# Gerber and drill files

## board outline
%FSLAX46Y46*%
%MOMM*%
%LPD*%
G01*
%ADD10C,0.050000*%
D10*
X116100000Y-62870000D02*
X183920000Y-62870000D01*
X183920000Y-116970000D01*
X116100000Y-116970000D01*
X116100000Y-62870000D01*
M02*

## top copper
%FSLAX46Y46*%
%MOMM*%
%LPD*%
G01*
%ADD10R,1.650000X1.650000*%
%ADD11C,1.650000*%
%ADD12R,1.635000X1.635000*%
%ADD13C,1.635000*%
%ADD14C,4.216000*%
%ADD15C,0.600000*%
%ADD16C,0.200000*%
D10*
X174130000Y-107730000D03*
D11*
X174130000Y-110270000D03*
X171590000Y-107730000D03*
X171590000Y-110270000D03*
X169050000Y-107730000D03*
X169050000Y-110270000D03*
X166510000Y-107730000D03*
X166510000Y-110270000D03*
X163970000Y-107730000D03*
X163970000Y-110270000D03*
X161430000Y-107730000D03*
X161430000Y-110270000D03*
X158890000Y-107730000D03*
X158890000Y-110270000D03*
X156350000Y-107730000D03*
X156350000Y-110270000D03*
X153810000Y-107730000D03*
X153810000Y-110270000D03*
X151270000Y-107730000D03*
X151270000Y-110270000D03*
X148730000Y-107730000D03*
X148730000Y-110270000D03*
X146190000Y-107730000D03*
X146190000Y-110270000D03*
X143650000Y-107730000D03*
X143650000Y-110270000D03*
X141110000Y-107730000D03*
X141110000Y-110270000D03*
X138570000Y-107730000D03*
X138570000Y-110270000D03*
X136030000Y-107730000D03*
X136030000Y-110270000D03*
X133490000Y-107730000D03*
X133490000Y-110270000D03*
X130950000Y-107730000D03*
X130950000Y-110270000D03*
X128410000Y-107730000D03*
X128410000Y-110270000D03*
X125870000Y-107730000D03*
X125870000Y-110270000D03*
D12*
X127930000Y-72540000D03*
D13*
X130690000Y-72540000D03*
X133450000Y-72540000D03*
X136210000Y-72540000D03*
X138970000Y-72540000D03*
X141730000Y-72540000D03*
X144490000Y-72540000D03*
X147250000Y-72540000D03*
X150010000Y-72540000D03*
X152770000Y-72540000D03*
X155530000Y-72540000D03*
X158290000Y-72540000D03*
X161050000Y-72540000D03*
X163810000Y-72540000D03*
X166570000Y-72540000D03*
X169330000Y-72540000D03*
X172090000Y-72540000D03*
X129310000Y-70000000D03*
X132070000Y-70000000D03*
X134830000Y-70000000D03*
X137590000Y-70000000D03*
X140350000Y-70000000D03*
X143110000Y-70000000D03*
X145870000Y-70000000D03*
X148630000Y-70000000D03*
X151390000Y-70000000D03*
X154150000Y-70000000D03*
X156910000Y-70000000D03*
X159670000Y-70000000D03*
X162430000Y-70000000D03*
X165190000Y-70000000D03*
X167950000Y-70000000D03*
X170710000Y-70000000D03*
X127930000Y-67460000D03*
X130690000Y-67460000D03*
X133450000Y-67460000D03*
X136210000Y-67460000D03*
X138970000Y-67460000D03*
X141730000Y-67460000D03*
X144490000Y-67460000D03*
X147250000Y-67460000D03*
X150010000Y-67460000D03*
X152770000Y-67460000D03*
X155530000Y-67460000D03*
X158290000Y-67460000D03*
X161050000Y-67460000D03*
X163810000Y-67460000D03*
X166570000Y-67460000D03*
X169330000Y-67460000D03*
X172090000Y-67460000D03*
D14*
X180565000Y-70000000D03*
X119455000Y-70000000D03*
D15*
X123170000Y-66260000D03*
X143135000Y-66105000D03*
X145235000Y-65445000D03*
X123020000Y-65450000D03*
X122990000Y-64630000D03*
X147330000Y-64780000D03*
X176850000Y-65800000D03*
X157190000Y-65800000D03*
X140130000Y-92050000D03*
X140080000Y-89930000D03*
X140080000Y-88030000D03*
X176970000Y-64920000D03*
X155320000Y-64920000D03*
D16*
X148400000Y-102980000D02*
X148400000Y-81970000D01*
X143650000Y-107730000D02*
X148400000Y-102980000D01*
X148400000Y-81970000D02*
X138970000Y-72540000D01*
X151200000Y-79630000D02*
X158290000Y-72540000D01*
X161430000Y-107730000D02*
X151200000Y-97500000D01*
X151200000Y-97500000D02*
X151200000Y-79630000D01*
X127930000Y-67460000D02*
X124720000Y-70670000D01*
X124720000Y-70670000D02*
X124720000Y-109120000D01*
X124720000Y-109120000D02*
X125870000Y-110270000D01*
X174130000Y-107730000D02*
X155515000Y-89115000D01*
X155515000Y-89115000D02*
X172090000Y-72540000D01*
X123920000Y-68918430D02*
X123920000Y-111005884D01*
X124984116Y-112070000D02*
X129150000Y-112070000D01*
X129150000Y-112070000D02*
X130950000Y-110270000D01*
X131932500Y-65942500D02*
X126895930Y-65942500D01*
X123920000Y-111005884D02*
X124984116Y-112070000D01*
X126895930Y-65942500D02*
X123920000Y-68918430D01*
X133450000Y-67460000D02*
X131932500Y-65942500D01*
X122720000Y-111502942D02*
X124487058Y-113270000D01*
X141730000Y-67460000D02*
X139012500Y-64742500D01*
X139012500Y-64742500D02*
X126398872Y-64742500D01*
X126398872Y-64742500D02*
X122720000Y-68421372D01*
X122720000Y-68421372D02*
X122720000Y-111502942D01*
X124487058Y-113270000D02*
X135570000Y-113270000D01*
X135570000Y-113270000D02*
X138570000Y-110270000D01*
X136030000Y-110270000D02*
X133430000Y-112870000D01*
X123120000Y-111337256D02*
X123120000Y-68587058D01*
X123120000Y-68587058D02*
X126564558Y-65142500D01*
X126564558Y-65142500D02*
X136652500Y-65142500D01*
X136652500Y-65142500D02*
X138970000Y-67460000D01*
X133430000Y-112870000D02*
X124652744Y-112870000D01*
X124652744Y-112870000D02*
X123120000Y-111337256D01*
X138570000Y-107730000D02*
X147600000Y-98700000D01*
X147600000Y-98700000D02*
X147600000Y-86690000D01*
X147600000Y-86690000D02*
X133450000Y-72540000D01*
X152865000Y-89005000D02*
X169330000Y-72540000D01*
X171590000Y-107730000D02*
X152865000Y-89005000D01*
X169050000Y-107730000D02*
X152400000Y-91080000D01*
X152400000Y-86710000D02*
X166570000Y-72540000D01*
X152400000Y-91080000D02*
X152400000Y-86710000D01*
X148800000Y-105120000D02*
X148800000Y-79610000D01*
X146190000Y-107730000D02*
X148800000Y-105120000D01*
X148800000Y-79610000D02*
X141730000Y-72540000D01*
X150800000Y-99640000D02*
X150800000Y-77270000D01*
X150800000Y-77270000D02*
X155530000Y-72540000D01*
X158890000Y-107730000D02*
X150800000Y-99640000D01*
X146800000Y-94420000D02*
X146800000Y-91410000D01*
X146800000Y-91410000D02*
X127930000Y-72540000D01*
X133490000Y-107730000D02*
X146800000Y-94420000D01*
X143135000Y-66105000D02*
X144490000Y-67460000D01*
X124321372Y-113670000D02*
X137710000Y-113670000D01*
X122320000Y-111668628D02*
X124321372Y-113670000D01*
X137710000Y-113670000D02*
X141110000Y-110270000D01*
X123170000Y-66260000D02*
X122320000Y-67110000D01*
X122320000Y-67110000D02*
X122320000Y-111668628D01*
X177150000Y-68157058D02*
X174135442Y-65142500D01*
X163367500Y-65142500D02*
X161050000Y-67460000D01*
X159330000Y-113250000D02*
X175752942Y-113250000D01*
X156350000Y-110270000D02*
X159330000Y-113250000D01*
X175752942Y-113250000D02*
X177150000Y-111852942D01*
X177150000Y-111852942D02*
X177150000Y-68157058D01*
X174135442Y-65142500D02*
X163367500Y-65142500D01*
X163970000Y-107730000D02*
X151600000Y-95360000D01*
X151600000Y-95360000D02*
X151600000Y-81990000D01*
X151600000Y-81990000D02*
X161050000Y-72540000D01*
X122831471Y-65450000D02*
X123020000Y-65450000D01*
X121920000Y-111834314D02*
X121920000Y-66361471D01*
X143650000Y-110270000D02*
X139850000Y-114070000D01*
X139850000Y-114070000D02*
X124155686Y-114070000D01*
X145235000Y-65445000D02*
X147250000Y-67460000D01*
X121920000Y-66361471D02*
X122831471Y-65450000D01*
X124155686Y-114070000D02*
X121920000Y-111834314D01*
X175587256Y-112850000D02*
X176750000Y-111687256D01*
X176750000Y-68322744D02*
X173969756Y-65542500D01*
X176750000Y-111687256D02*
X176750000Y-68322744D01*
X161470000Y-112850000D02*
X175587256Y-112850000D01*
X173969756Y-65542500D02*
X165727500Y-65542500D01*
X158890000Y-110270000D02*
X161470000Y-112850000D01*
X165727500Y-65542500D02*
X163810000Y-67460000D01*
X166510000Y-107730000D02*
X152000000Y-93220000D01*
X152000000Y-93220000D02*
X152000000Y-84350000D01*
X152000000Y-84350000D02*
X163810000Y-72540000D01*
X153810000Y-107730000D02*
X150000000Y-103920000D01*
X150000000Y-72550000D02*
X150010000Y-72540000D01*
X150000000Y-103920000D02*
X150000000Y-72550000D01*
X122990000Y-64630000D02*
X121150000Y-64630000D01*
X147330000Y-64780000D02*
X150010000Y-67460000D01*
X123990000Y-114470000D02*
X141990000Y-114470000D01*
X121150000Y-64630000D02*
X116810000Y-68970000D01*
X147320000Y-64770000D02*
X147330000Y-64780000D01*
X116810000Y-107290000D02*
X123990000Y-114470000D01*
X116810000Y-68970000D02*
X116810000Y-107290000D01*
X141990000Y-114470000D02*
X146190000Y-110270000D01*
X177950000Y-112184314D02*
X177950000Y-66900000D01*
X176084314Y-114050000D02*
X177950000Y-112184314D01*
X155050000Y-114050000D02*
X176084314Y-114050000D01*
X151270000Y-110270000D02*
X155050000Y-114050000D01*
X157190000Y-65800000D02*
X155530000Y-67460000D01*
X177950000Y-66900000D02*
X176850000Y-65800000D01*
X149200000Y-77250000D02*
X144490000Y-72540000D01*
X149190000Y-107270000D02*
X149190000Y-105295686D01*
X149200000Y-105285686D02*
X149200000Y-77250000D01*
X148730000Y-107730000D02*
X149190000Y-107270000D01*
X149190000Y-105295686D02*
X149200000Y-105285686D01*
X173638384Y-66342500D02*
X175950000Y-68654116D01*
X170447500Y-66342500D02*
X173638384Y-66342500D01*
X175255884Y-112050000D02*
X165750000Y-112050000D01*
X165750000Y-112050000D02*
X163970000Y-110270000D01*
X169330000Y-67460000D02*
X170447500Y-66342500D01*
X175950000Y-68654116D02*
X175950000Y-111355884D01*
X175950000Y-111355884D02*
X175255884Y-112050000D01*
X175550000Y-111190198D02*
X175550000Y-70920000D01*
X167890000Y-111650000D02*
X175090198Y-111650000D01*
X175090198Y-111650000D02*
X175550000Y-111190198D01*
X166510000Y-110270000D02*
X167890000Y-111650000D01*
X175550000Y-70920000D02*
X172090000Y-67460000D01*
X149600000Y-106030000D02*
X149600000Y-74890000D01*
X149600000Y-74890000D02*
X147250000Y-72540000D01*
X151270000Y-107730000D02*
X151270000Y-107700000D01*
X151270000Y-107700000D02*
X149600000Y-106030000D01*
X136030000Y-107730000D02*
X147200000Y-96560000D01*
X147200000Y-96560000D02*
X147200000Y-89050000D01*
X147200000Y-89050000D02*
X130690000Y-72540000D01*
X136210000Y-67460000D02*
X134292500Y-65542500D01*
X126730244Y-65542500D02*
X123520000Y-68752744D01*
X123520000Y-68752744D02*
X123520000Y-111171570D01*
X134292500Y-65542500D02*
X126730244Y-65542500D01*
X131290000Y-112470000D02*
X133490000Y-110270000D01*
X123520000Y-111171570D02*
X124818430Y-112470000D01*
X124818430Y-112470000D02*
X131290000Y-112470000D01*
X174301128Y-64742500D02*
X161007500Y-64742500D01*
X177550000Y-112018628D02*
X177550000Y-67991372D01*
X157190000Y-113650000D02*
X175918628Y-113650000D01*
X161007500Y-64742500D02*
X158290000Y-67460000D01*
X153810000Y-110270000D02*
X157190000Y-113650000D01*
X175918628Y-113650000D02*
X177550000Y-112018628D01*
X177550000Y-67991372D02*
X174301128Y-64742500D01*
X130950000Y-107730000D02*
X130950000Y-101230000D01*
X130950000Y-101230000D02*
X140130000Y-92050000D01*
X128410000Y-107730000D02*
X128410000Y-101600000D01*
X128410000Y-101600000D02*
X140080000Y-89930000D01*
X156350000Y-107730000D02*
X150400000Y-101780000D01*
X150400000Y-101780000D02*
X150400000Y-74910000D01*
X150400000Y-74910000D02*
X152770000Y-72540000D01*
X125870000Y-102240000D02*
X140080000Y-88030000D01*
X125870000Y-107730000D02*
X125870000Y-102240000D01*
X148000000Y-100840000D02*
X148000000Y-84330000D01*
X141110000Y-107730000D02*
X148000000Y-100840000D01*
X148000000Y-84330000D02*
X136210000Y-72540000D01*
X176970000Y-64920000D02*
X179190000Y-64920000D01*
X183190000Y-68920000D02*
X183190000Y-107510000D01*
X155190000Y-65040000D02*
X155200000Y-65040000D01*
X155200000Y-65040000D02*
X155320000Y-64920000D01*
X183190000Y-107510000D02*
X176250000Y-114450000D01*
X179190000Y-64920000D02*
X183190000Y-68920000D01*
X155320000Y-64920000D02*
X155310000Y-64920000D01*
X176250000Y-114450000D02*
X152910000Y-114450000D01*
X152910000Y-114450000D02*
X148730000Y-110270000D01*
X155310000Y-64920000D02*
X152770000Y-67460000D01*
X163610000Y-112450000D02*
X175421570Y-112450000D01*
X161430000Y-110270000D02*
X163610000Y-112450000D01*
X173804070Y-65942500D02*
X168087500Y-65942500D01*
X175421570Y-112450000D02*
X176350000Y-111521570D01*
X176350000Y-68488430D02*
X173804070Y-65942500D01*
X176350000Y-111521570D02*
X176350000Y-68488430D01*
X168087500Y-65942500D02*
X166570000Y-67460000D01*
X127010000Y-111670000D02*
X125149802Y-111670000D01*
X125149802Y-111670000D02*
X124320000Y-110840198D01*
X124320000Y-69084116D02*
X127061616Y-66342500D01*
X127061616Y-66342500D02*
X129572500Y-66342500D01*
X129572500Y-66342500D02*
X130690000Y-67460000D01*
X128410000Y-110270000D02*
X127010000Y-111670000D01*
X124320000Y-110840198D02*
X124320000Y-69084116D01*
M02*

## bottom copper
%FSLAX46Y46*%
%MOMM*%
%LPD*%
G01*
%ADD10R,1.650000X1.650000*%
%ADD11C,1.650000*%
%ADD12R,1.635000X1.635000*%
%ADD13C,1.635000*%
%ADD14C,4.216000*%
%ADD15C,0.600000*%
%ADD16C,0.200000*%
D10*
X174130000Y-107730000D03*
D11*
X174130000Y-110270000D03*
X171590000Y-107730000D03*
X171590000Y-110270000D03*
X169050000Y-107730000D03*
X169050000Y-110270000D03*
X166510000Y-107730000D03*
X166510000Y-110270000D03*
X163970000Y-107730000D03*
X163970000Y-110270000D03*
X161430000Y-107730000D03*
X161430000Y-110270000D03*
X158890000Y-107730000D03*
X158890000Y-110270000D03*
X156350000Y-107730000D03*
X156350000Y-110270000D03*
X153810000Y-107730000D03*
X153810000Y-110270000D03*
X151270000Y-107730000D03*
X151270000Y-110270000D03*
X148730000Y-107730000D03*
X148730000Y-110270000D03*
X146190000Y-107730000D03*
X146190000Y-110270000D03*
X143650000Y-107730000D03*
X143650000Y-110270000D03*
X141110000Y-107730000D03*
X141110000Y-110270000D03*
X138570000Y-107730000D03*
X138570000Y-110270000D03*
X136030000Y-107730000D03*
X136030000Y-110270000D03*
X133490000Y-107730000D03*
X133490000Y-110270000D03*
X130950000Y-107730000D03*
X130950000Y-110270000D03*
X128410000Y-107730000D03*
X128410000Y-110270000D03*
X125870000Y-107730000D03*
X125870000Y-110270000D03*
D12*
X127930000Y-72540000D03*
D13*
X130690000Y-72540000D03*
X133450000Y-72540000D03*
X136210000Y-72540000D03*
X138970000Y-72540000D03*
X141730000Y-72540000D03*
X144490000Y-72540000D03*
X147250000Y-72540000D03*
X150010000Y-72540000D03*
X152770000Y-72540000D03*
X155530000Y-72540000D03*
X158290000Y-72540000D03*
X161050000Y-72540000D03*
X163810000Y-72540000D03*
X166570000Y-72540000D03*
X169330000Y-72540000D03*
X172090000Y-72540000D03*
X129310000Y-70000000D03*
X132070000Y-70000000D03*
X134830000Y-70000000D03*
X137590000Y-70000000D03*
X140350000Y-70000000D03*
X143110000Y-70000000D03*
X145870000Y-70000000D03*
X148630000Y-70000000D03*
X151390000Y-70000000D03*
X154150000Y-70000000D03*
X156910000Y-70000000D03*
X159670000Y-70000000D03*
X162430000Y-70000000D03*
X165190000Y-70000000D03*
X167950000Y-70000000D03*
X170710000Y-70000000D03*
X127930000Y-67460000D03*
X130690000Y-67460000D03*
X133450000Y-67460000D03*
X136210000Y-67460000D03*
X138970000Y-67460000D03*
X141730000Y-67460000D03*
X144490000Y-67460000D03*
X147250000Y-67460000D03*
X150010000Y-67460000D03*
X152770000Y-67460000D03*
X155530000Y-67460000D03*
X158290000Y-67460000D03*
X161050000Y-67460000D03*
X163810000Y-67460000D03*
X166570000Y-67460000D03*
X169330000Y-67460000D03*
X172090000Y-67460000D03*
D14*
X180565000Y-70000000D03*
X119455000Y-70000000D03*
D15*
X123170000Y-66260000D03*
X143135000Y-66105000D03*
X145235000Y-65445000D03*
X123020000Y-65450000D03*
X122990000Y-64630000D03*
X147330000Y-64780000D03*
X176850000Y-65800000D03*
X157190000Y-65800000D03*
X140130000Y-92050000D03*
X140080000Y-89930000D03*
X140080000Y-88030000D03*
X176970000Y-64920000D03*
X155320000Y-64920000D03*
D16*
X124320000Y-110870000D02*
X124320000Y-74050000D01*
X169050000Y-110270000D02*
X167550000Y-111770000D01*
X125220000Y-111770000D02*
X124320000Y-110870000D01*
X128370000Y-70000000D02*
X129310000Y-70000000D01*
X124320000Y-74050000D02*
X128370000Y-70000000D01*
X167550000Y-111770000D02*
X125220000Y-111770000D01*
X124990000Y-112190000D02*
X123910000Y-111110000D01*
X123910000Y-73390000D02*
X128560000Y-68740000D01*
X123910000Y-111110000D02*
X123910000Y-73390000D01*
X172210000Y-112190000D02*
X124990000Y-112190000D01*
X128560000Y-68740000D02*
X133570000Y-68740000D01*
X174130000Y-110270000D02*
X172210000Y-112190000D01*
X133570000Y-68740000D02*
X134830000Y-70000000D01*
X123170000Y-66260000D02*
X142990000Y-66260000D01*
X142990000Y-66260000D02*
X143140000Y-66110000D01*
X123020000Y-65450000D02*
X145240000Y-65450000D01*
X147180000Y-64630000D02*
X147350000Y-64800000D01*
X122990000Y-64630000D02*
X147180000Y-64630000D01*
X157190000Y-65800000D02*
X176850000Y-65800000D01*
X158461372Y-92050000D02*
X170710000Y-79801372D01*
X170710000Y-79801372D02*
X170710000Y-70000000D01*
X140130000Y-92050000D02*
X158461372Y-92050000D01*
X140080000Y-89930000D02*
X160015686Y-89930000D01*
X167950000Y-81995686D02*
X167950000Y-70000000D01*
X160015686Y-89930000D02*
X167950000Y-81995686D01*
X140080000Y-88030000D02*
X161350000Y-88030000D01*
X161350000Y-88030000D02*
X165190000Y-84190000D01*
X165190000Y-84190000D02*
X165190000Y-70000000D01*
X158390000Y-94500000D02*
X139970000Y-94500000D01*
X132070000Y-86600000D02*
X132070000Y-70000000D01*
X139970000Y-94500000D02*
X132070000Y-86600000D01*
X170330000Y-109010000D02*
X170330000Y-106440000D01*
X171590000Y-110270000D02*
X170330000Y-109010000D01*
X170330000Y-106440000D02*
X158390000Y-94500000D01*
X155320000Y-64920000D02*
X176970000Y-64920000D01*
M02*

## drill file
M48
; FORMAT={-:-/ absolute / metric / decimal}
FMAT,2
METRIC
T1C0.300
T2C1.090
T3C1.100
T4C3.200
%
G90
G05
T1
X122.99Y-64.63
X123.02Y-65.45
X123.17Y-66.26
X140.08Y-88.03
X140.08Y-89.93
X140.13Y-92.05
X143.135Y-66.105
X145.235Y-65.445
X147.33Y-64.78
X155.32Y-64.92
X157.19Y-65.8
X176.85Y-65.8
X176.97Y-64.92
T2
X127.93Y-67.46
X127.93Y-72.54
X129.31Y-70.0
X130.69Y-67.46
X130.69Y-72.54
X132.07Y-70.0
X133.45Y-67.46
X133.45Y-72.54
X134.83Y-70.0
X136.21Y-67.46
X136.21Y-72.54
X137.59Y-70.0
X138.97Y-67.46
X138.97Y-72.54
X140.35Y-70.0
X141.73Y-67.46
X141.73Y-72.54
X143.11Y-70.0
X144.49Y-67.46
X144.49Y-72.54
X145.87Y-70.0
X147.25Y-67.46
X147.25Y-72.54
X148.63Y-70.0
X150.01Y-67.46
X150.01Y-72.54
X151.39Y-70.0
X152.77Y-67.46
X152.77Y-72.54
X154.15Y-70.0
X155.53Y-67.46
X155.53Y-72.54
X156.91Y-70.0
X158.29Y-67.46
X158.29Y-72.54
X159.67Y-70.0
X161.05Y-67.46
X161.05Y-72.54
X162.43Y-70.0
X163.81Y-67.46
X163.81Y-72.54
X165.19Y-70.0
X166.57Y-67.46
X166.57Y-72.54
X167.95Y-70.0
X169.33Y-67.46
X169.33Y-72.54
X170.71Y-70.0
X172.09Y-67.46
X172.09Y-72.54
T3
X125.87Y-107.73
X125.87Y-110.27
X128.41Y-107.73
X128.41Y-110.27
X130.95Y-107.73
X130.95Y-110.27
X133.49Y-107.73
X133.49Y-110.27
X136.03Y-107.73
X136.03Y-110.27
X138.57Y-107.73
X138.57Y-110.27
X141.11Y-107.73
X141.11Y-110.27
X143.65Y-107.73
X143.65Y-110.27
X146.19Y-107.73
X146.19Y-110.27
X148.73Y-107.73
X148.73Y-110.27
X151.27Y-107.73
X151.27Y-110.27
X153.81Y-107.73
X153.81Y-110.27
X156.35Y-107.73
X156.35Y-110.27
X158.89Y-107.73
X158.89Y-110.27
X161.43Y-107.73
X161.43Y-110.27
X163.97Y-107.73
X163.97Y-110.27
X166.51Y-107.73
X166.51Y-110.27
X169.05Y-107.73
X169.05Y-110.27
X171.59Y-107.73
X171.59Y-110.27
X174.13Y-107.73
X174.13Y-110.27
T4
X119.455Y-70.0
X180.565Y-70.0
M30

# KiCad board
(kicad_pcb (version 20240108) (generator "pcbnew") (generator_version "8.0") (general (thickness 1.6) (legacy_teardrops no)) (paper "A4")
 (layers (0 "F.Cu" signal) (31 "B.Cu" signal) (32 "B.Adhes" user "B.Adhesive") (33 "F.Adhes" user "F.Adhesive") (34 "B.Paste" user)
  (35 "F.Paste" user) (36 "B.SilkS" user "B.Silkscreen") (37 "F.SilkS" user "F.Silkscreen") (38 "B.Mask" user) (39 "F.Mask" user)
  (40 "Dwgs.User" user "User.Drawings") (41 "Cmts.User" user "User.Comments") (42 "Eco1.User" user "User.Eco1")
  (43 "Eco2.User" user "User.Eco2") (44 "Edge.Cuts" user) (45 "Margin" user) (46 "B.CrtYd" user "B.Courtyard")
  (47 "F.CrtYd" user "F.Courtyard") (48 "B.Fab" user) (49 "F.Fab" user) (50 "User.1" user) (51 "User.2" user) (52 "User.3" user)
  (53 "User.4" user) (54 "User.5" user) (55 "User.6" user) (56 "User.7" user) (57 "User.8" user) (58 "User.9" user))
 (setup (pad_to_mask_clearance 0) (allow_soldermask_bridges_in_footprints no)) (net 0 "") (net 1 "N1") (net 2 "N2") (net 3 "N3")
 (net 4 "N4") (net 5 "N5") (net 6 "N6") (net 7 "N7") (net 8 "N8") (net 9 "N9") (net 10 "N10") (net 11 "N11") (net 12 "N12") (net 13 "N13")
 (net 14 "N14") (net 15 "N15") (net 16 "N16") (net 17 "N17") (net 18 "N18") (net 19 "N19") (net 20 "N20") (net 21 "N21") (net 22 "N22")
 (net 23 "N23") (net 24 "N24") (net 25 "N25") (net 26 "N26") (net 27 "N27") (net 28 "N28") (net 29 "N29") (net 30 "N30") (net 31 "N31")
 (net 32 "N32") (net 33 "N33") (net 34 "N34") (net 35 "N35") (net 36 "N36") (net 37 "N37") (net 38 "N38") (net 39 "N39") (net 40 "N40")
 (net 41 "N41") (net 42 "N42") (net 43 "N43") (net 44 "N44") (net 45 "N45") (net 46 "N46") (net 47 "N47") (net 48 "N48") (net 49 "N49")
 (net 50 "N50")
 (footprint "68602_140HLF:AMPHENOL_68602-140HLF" (layer "F.Cu") (at 150 109 180)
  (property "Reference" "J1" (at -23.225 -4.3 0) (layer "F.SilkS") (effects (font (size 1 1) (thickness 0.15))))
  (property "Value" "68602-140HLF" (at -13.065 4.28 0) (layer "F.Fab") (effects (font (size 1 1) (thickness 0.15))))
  (pad "01" thru_hole rect (at -24.13 1.27 180) (size 1.65 1.65) (drill 1.1) (layers "*.Cu" "*.Mask") (remove_unused_layers no) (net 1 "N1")
   (solder_mask_margin 0.102))
  (pad "02" thru_hole circle (at -24.13 -1.27 180) (size 1.65 1.65) (drill 1.1) (layers "*.Cu" "*.Mask") (remove_unused_layers no)
   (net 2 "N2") (solder_mask_margin 0.102))
  (pad "03" thru_hole circle (at -21.59 1.27 180) (size 1.65 1.65) (drill 1.1) (layers "*.Cu" "*.Mask") (remove_unused_layers no)
   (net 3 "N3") (solder_mask_margin 0.102))
  (pad "04" thru_hole circle (at -21.59 -1.27 180) (size 1.65 1.65) (drill 1.1) (layers "*.Cu" "*.Mask") (remove_unused_layers no)
   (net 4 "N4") (solder_mask_margin 0.102))
  (pad "05" thru_hole circle (at -19.05 1.27 180) (size 1.65 1.65) (drill 1.1) (layers "*.Cu" "*.Mask") (remove_unused_layers no)
   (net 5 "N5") (solder_mask_margin 0.102))
  (pad "06" thru_hole circle (at -19.05 -1.27 180) (size 1.65 1.65) (drill 1.1) (layers "*.Cu" "*.Mask") (remove_unused_layers no)
   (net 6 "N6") (solder_mask_margin 0.102))
  (pad "07" thru_hole circle (at -16.51 1.27 180) (size 1.65 1.65) (drill 1.1) (layers "*.Cu" "*.Mask") (remove_unused_layers no)
   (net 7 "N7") (solder_mask_margin 0.102))
  (pad "08" thru_hole circle (at -16.51 -1.27 180) (size 1.65 1.65) (drill 1.1) (layers "*.Cu" "*.Mask") (remove_unused_layers no)
   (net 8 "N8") (solder_mask_margin 0.102))
  (pad "09" thru_hole circle (at -13.97 1.27 180) (size 1.65 1.65) (drill 1.1) (layers "*.Cu" "*.Mask") (remove_unused_layers no)
   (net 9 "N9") (solder_mask_margin 0.102))
  (pad "10" thru_hole circle (at -13.97 -1.27 180) (size 1.65 1.65) (drill 1.1) (layers "*.Cu" "*.Mask") (remove_unused_layers no)
   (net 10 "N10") (solder_mask_margin 0.102))
  (pad "11" thru_hole circle (at -11.43 1.27 180) (size 1.65 1.65) (drill 1.1) (layers "*.Cu" "*.Mask") (remove_unused_layers no)
   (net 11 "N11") (solder_mask_margin 0.102))
  (pad "12" thru_hole circle (at -11.43 -1.27 180) (size 1.65 1.65) (drill 1.1) (layers "*.Cu" "*.Mask") (remove_unused_layers no)
   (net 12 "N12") (solder_mask_margin 0.102))
  (pad "13" thru_hole circle (at -8.89 1.27 180) (size 1.65 1.65) (drill 1.1) (layers "*.Cu" "*.Mask") (remove_unused_layers no)
   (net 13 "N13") (solder_mask_margin 0.102))
  (pad "14" thru_hole circle (at -8.89 -1.27 180) (size 1.65 1.65) (drill 1.1) (layers "*.Cu" "*.Mask") (remove_unused_layers no)
   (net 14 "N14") (solder_mask_margin 0.102))
  (pad "15" thru_hole circle (at -6.35 1.27 180) (size 1.65 1.65) (drill 1.1) (layers "*.Cu" "*.Mask") (remove_unused_layers no)
   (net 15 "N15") (solder_mask_margin 0.102))
  (pad "16" thru_hole circle (at -6.35 -1.27 180) (size 1.65 1.65) (drill 1.1) (layers "*.Cu" "*.Mask") (remove_unused_layers no)
   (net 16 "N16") (solder_mask_margin 0.102))
  (pad "17" thru_hole circle (at -3.81 1.27 180) (size 1.65 1.65) (drill 1.1) (layers "*.Cu" "*.Mask") (remove_unused_layers no)
   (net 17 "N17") (solder_mask_margin 0.102))
  (pad "18" thru_hole circle (at -3.81 -1.27 180) (size 1.65 1.65) (drill 1.1) (layers "*.Cu" "*.Mask") (remove_unused_layers no)
   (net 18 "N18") (solder_mask_margin 0.102))
  (pad "19" thru_hole circle (at -1.27 1.27 180) (size 1.65 1.65) (drill 1.1) (layers "*.Cu" "*.Mask") (remove_unused_layers no)
   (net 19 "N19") (solder_mask_margin 0.102))
  (pad "20" thru_hole circle (at -1.27 -1.27 180) (size 1.65 1.65) (drill 1.1) (layers "*.Cu" "*.Mask") (remove_unused_layers no)
   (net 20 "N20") (solder_mask_margin 0.102))
  (pad "21" thru_hole circle (at 1.27 1.27 180) (size 1.65 1.65) (drill 1.1) (layers "*.Cu" "*.Mask") (remove_unused_layers no)
   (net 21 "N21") (solder_mask_margin 0.102))
  (pad "22" thru_hole circle (at 1.27 -1.27 180) (size 1.65 1.65) (drill 1.1) (layers "*.Cu" "*.Mask") (remove_unused_layers no)
   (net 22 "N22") (solder_mask_margin 0.102))
  (pad "23" thru_hole circle (at 3.81 1.27 180) (size 1.65 1.65) (drill 1.1) (layers "*.Cu" "*.Mask") (remove_unused_layers no)
   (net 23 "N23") (solder_mask_margin 0.102))
  (pad "24" thru_hole circle (at 3.81 -1.27 180) (size 1.65 1.65) (drill 1.1) (layers "*.Cu" "*.Mask") (remove_unused_layers no)
   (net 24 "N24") (solder_mask_margin 0.102))
  (pad "25" thru_hole circle (at 6.35 1.27 180) (size 1.65 1.65) (drill 1.1) (layers "*.Cu" "*.Mask") (remove_unused_layers no)
   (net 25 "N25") (solder_mask_margin 0.102))
  (pad "26" thru_hole circle (at 6.35 -1.27 180) (size 1.65 1.65) (drill 1.1) (layers "*.Cu" "*.Mask") (remove_unused_layers no)
   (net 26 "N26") (solder_mask_margin 0.102))
  (pad "27" thru_hole circle (at 8.89 1.27 180) (size 1.65 1.65) (drill 1.1) (layers "*.Cu" "*.Mask") (remove_unused_layers no)
   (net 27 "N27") (solder_mask_margin 0.102))
  (pad "28" thru_hole circle (at 8.89 -1.27 180) (size 1.65 1.65) (drill 1.1) (layers "*.Cu" "*.Mask") (remove_unused_layers no)
   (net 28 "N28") (solder_mask_margin 0.102))
  (pad "29" thru_hole circle (at 11.43 1.27 180) (size 1.65 1.65) (drill 1.1) (layers "*.Cu" "*.Mask") (remove_unused_layers no)
   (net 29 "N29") (solder_mask_margin 0.102))
  (pad "30" thru_hole circle (at 11.43 -1.27 180) (size 1.65 1.65) (drill 1.1) (layers "*.Cu" "*.Mask") (remove_unused_layers no)
   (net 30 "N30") (solder_mask_margin 0.102))
  (pad "31" thru_hole circle (at 13.97 1.27 180) (size 1.65 1.65) (drill 1.1) (layers "*.Cu" "*.Mask") (remove_unused_layers no)
   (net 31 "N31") (solder_mask_margin 0.102))
  (pad "32" thru_hole circle (at 13.97 -1.27 180) (size 1.65 1.65) (drill 1.1) (layers "*.Cu" "*.Mask") (remove_unused_layers no)
   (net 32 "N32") (solder_mask_margin 0.102))
  (pad "33" thru_hole circle (at 16.51 1.27 180) (size 1.65 1.65) (drill 1.1) (layers "*.Cu" "*.Mask") (remove_unused_layers no)
   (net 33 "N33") (solder_mask_margin 0.102))
  (pad "34" thru_hole circle (at 16.51 -1.27 180) (size 1.65 1.65) (drill 1.1) (layers "*.Cu" "*.Mask") (remove_unused_layers no)
   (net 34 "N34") (solder_mask_margin 0.102))
  (pad "35" thru_hole circle (at 19.05 1.27 180) (size 1.65 1.65) (drill 1.1) (layers "*.Cu" "*.Mask") (remove_unused_layers no)
   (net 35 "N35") (solder_mask_margin 0.102))
  (pad "36" thru_hole circle (at 19.05 -1.27 180) (size 1.65 1.65) (drill 1.1) (layers "*.Cu" "*.Mask") (remove_unused_layers no)
   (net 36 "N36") (solder_mask_margin 0.102))
  (pad "37" thru_hole circle (at 21.59 1.27 180) (size 1.65 1.65) (drill 1.1) (layers "*.Cu" "*.Mask") (remove_unused_layers no)
   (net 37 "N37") (solder_mask_margin 0.102))
  (pad "38" thru_hole circle (at 21.59 -1.27 180) (size 1.65 1.65) (drill 1.1) (layers "*.Cu" "*.Mask") (remove_unused_layers no)
   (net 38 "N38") (solder_mask_margin 0.102))
  (pad "39" thru_hole circle (at 24.13 1.27 180) (size 1.65 1.65) (drill 1.1) (layers "*.Cu" "*.Mask") (remove_unused_layers no)
   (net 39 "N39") (solder_mask_margin 0.102))
  (pad "40" thru_hole circle (at 24.13 -1.27 180) (size 1.65 1.65) (drill 1.1) (layers "*.Cu" "*.Mask") (remove_unused_layers no)
   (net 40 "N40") (solder_mask_margin 0.102)))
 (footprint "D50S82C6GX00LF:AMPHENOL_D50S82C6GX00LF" (layer "F.Cu") (at 150.01 70 180)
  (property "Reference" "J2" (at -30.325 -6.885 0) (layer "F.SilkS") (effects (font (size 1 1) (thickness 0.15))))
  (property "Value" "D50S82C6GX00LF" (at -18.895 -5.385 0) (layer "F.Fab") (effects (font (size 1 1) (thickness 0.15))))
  (pad "1" thru_hole rect (at 22.08 -2.54 180) (size 1.635 1.635) (drill 1.09) (layers "*.Cu" "*.Mask") (remove_unused_layers no)
   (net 33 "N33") (solder_mask_margin 0.102))
  (pad "2" thru_hole circle (at 19.32 -2.54 180) (size 1.635 1.635) (drill 1.09) (layers "*.Cu" "*.Mask") (remove_unused_layers no)
   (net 31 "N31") (solder_mask_margin 0.102))
  (pad "3" thru_hole circle (at 16.56 -2.54 180) (size 1.635 1.635) (drill 1.09) (layers "*.Cu" "*.Mask") (remove_unused_layers no)
   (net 29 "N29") (solder_mask_margin 0.102))
  (pad "4" thru_hole circle (at 13.8 -2.54 180) (size 1.635 1.635) (drill 1.09) (layers "*.Cu" "*.Mask") (remove_unused_layers no)
   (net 27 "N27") (solder_mask_margin 0.102))
  (pad "5" thru_hole circle (at 11.04 -2.54 180) (size 1.635 1.635) (drill 1.09) (layers "*.Cu" "*.Mask") (remove_unused_layers no)
   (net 25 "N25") (solder_mask_margin 0.102))
  (pad "6" thru_hole circle (at 8.28 -2.54 180) (size 1.635 1.635) (drill 1.09) (layers "*.Cu" "*.Mask") (remove_unused_layers no)
   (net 23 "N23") (solder_mask_margin 0.102))
  (pad "7" thru_hole circle (at 5.52 -2.54 180) (size 1.635 1.635) (drill 1.09) (layers "*.Cu" "*.Mask") (remove_unused_layers no)
   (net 21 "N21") (solder_mask_margin 0.102))
  (pad "8" thru_hole circle (at 2.76 -2.54 180) (size 1.635 1.635) (drill 1.09) (layers "*.Cu" "*.Mask") (remove_unused_layers no)
   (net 19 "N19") (solder_mask_margin 0.102))
  (pad "9" thru_hole circle (at 0 -2.54 180) (size 1.635 1.635) (drill 1.09) (layers "*.Cu" "*.Mask") (remove_unused_layers no)
   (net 17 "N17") (solder_mask_margin 0.102))
  (pad "10" thru_hole circle (at -2.76 -2.54 180) (size 1.635 1.635) (drill 1.09) (layers "*.Cu" "*.Mask") (remove_unused_layers no)
   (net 15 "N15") (solder_mask_margin 0.102))
  (pad "11" thru_hole circle (at -5.52 -2.54 180) (size 1.635 1.635) (drill 1.09) (layers "*.Cu" "*.Mask") (remove_unused_layers no)
   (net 13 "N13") (solder_mask_margin 0.102))
  (pad "12" thru_hole circle (at -8.28 -2.54 180) (size 1.635 1.635) (drill 1.09) (layers "*.Cu" "*.Mask") (remove_unused_layers no)
   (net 11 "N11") (solder_mask_margin 0.102))
  (pad "13" thru_hole circle (at -11.04 -2.54 180) (size 1.635 1.635) (drill 1.09) (layers "*.Cu" "*.Mask") (remove_unused_layers no)
   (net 9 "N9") (solder_mask_margin 0.102))
  (pad "14" thru_hole circle (at -13.8 -2.54 180) (size 1.635 1.635) (drill 1.09) (layers "*.Cu" "*.Mask") (remove_unused_layers no)
   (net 7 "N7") (solder_mask_margin 0.102))
  (pad "15" thru_hole circle (at -16.56 -2.54 180) (size 1.635 1.635) (drill 1.09) (layers "*.Cu" "*.Mask") (remove_unused_layers no)
   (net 5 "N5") (solder_mask_margin 0.102))
  (pad "16" thru_hole circle (at -19.32 -2.54 180) (size 1.635 1.635) (drill 1.09) (layers "*.Cu" "*.Mask") (remove_unused_layers no)
   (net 3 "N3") (solder_mask_margin 0.102))
  (pad "17" thru_hole circle (at -22.08 -2.54 180) (size 1.635 1.635) (drill 1.09) (layers "*.Cu" "*.Mask") (remove_unused_layers no)
   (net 1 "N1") (solder_mask_margin 0.102))
  (pad "18" thru_hole circle (at 20.7 0 180) (size 1.635 1.635) (drill 1.09) (layers "*.Cu" "*.Mask") (remove_unused_layers no) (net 6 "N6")
   (solder_mask_margin 0.102))
  (pad "19" thru_hole circle (at 17.94 0 180) (size 1.635 1.635) (drill 1.09) (layers "*.Cu" "*.Mask") (remove_unused_layers no)
   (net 4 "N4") (solder_mask_margin 0.102))
  (pad "20" thru_hole circle (at 15.18 0 180) (size 1.635 1.635) (drill 1.09) (layers "*.Cu" "*.Mask") (remove_unused_layers no)
   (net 2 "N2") (solder_mask_margin 0.102))
  (pad "21" thru_hole circle (at 12.42 0 180) (size 1.635 1.635) (drill 1.09) (layers "*.Cu" "*.Mask") (remove_unused_layers no)
   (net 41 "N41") (solder_mask_margin 0.102))
  (pad "22" thru_hole circle (at 9.66 0 180) (size 1.635 1.635) (drill 1.09) (layers "*.Cu" "*.Mask") (remove_unused_layers no)
   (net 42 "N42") (solder_mask_margin 0.102))
  (pad "23" thru_hole circle (at 6.9 0 180) (size 1.635 1.635) (drill 1.09) (layers "*.Cu" "*.Mask") (remove_unused_layers no)
   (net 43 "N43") (solder_mask_margin 0.102))
  (pad "24" thru_hole circle (at 4.14 0 180) (size 1.635 1.635) (drill 1.09) (layers "*.Cu" "*.Mask") (remove_unused_layers no)
   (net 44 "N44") (solder_mask_margin 0.102))
  (pad "25" thru_hole circle (at 1.38 0 180) (size 1.635 1.635) (drill 1.09) (layers "*.Cu" "*.Mask") (remove_unused_layers no)
   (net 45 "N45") (solder_mask_margin 0.102))
  (pad "26" thru_hole circle (at -1.38 0 180) (size 1.635 1.635) (drill 1.09) (layers "*.Cu" "*.Mask") (remove_unused_layers no)
   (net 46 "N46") (solder_mask_margin 0.102))
  (pad "27" thru_hole circle (at -4.14 0 180) (size 1.635 1.635) (drill 1.09) (layers "*.Cu" "*.Mask") (remove_unused_layers no)
   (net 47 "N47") (solder_mask_margin 0.102))
  (pad "28" thru_hole circle (at -6.9 0 180) (size 1.635 1.635) (drill 1.09) (layers "*.Cu" "*.Mask") (remove_unused_layers no)
   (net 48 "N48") (solder_mask_margin 0.102))
  (pad "29" thru_hole circle (at -9.66 0 180) (size 1.635 1.635) (drill 1.09) (layers "*.Cu" "*.Mask") (remove_unused_layers no)
   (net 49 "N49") (solder_mask_margin 0.102))
  (pad "30" thru_hole circle (at -12.42 0 180) (size 1.635 1.635) (drill 1.09) (layers "*.Cu" "*.Mask") (remove_unused_layers no)
   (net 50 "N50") (solder_mask_margin 0.102))
  (pad "31" thru_hole circle (at -15.18 0 180) (size 1.635 1.635) (drill 1.09) (layers "*.Cu" "*.Mask") (remove_unused_layers no)
   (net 39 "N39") (solder_mask_margin 0.102))
  (pad "32" thru_hole circle (at -17.94 0 180) (size 1.635 1.635) (drill 1.09) (layers "*.Cu" "*.Mask") (remove_unused_layers no)
   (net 37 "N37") (solder_mask_margin 0.102))
  (pad "33" thru_hole circle (at -20.7 0 180) (size 1.635 1.635) (drill 1.09) (layers "*.Cu" "*.Mask") (remove_unused_layers no)
   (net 35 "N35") (solder_mask_margin 0.102))
  (pad "34" thru_hole circle (at 22.08 2.54 180) (size 1.635 1.635) (drill 1.09) (layers "*.Cu" "*.Mask") (remove_unused_layers no)
   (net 40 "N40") (solder_mask_margin 0.102))
  (pad "35" thru_hole circle (at 19.32 2.54 180) (size 1.635 1.635) (drill 1.09) (layers "*.Cu" "*.Mask") (remove_unused_layers no)
   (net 38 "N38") (solder_mask_margin 0.102))
  (pad "36" thru_hole circle (at 16.56 2.54 180) (size 1.635 1.635) (drill 1.09) (layers "*.Cu" "*.Mask") (remove_unused_layers no)
   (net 36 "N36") (solder_mask_margin 0.102))
  (pad "37" thru_hole circle (at 13.8 2.54 180) (size 1.635 1.635) (drill 1.09) (layers "*.Cu" "*.Mask") (remove_unused_layers no)
   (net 34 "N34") (solder_mask_margin 0.102))
  (pad "38" thru_hole circle (at 11.04 2.54 180) (size 1.635 1.635) (drill 1.09) (layers "*.Cu" "*.Mask") (remove_unused_layers no)
   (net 32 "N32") (solder_mask_margin 0.102))
  (pad "39" thru_hole circle (at 8.28 2.54 180) (size 1.635 1.635) (drill 1.09) (layers "*.Cu" "*.Mask") (remove_unused_layers no)
   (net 30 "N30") (solder_mask_margin 0.102))
  (pad "40" thru_hole circle (at 5.52 2.54 180) (size 1.635 1.635) (drill 1.09) (layers "*.Cu" "*.Mask") (remove_unused_layers no)
   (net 28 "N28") (solder_mask_margin 0.102))
  (pad "41" thru_hole circle (at 2.76 2.54 180) (size 1.635 1.635) (drill 1.09) (layers "*.Cu" "*.Mask") (remove_unused_layers no)
   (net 26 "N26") (solder_mask_margin 0.102))
  (pad "42" thru_hole circle (at 0 2.54 180) (size 1.635 1.635) (drill 1.09) (layers "*.Cu" "*.Mask") (remove_unused_layers no)
   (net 24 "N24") (solder_mask_margin 0.102))
  (pad "43" thru_hole circle (at -2.76 2.54 180) (size 1.635 1.635) (drill 1.09) (layers "*.Cu" "*.Mask") (remove_unused_layers no)
   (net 22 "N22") (solder_mask_margin 0.102))
  (pad "44" thru_hole circle (at -5.52 2.54 180) (size 1.635 1.635) (drill 1.09) (layers "*.Cu" "*.Mask") (remove_unused_layers no)
   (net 20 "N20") (solder_mask_margin 0.102))
  (pad "45" thru_hole circle (at -8.28 2.54 180) (size 1.635 1.635) (drill 1.09) (layers "*.Cu" "*.Mask") (remove_unused_layers no)
   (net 18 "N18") (solder_mask_margin 0.102))
  (pad "46" thru_hole circle (at -11.04 2.54 180) (size 1.635 1.635) (drill 1.09) (layers "*.Cu" "*.Mask") (remove_unused_layers no)
   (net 16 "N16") (solder_mask_margin 0.102))
  (pad "47" thru_hole circle (at -13.8 2.54 180) (size 1.635 1.635) (drill 1.09) (layers "*.Cu" "*.Mask") (remove_unused_layers no)
   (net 14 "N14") (solder_mask_margin 0.102))
  (pad "48" thru_hole circle (at -16.56 2.54 180) (size 1.635 1.635) (drill 1.09) (layers "*.Cu" "*.Mask") (remove_unused_layers no)
   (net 12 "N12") (solder_mask_margin 0.102))
  (pad "49" thru_hole circle (at -19.32 2.54 180) (size 1.635 1.635) (drill 1.09) (layers "*.Cu" "*.Mask") (remove_unused_layers no)
   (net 10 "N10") (solder_mask_margin 0.102))
  (pad "50" thru_hole circle (at -22.08 2.54 180) (size 1.635 1.635) (drill 1.09) (layers "*.Cu" "*.Mask") (remove_unused_layers no)
   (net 8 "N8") (solder_mask_margin 0.102))
  (pad "SH1" thru_hole circle (at -30.555 0 180) (size 4.216 4.216) (drill 3.2) (layers "*.Cu" "*.Mask") (remove_unused_layers no)
   (solder_mask_margin 0.102))
  (pad "SH2" thru_hole circle (at 30.555 0 180) (size 4.216 4.216) (drill 3.2) (layers "*.Cu" "*.Mask") (remove_unused_layers no)
   (solder_mask_margin 0.102)))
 (gr_rect (start 116.1 62.87) (end 183.92 116.97) (stroke (width 0.05) (type default)) (fill none) (layer "Edge.Cuts"))
 (segment (start 148.4 102.98) (end 148.4 81.97) (width 0.2) (layer "F.Cu") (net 25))
 (segment (start 143.65 107.73) (end 148.4 102.98) (width 0.2) (layer "F.Cu") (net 25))
 (segment (start 148.4 81.97) (end 138.97 72.54) (width 0.2) (layer "F.Cu") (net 25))
 (segment (start 124.32 110.87) (end 124.32 74.05) (width 0.2) (layer "B.Cu") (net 6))
 (segment (start 169.05 110.27) (end 167.55 111.77) (width 0.2) (layer "B.Cu") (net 6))
 (segment (start 125.22 111.77) (end 124.32 110.87) (width 0.2) (layer "B.Cu") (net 6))
 (segment (start 128.37 70) (end 129.31 70) (width 0.2) (layer "B.Cu") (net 6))
 (segment (start 124.32 74.05) (end 128.37 70) (width 0.2) (layer "B.Cu") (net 6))
 (segment (start 167.55 111.77) (end 125.22 111.77) (width 0.2) (layer "B.Cu") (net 6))
 (segment (start 151.2 79.63) (end 158.29 72.54) (width 0.2) (layer "F.Cu") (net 11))
 (segment (start 161.43 107.73) (end 151.2 97.5) (width 0.2) (layer "F.Cu") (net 11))
 (segment (start 151.2 97.5) (end 151.2 79.63) (width 0.2) (layer "F.Cu") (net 11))
 (segment (start 127.93 67.46) (end 124.72 70.67) (width 0.2) (layer "F.Cu") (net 40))
 (segment (start 124.72 70.67) (end 124.72 109.12) (width 0.2) (layer "F.Cu") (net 40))
 (segment (start 124.72 109.12) (end 125.87 110.27) (width 0.2) (layer "F.Cu") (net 40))
 (segment (start 174.13 107.73) (end 155.515 89.115) (width 0.2) (layer "F.Cu") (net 1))
 (segment (start 155.515 89.115) (end 172.09 72.54) (width 0.2) (layer "F.Cu") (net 1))
 (segment (start 123.92 68.91843) (end 123.92 111.005884) (width 0.2) (layer "F.Cu") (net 36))
 (segment (start 124.984116 112.07) (end 129.15 112.07) (width 0.2) (layer "F.Cu") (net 36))
 (segment (start 129.15 112.07) (end 130.95 110.27) (width 0.2) (layer "F.Cu") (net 36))
 (segment (start 131.9325 65.9425) (end 126.89593 65.9425) (width 0.2) (layer "F.Cu") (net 36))
 (segment (start 123.92 111.005884) (end 124.984116 112.07) (width 0.2) (layer "F.Cu") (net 36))
 (segment (start 126.89593 65.9425) (end 123.92 68.91843) (width 0.2) (layer "F.Cu") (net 36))
 (segment (start 133.45 67.46) (end 131.9325 65.9425) (width 0.2) (layer "F.Cu") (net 36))
 (segment (start 122.72 111.502942) (end 124.487058 113.27) (width 0.2) (layer "F.Cu") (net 30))
 (segment (start 141.73 67.46) (end 139.0125 64.7425) (width 0.2) (layer "F.Cu") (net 30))
 (segment (start 139.0125 64.7425) (end 126.398872 64.7425) (width 0.2) (layer "F.Cu") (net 30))
 (segment (start 126.398872 64.7425) (end 122.72 68.421372) (width 0.2) (layer "F.Cu") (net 30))
 (segment (start 122.72 68.421372) (end 122.72 111.502942) (width 0.2) (layer "F.Cu") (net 30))
 (segment (start 124.487058 113.27) (end 135.57 113.27) (width 0.2) (layer "F.Cu") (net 30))
 (segment (start 135.57 113.27) (end 138.57 110.27) (width 0.2) (layer "F.Cu") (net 30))
 (segment (start 136.03 110.27) (end 133.43 112.87) (width 0.2) (layer "F.Cu") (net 32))
 (segment (start 123.12 111.337256) (end 123.12 68.587058) (width 0.2) (layer "F.Cu") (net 32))
 (segment (start 123.12 68.587058) (end 126.564558 65.1425) (width 0.2) (layer "F.Cu") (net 32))
 (segment (start 126.564558 65.1425) (end 136.6525 65.1425) (width 0.2) (layer "F.Cu") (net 32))
 (segment (start 136.6525 65.1425) (end 138.97 67.46) (width 0.2) (layer "F.Cu") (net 32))
 (segment (start 133.43 112.87) (end 124.652744 112.87) (width 0.2) (layer "F.Cu") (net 32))
 (segment (start 124.652744 112.87) (end 123.12 111.337256) (width 0.2) (layer "F.Cu") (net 32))
 (segment (start 138.57 107.73) (end 147.6 98.7) (width 0.2) (layer "F.Cu") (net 29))
 (segment (start 147.6 98.7) (end 147.6 86.69) (width 0.2) (layer "F.Cu") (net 29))
 (segment (start 147.6 86.69) (end 133.45 72.54) (width 0.2) (layer "F.Cu") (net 29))
 (segment (start 124.99 112.19) (end 123.91 111.11) (width 0.2) (layer "B.Cu") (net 2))
 (segment (start 123.91 73.39) (end 128.56 68.74) (width 0.2) (layer "B.Cu") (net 2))
 (segment (start 123.91 111.11) (end 123.91 73.39) (width 0.2) (layer "B.Cu") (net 2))
 (segment (start 172.21 112.19) (end 124.99 112.19) (width 0.2) (layer "B.Cu") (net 2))
 (segment (start 128.56 68.74) (end 133.57 68.74) (width 0.2) (layer "B.Cu") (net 2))
 (segment (start 174.13 110.27) (end 172.21 112.19) (width 0.2) (layer "B.Cu") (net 2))
 (segment (start 133.57 68.74) (end 134.83 70) (width 0.2) (layer "B.Cu") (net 2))
 (segment (start 152.865 89.005) (end 169.33 72.54) (width 0.2) (layer "F.Cu") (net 3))
 (segment (start 171.59 107.73) (end 152.865 89.005) (width 0.2) (layer "F.Cu") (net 3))
 (segment (start 169.05 107.73) (end 152.4 91.08) (width 0.2) (layer "F.Cu") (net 5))
 (segment (start 152.4 86.71) (end 166.57 72.54) (width 0.2) (layer "F.Cu") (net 5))
 (segment (start 152.4 91.08) (end 152.4 86.71) (width 0.2) (layer "F.Cu") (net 5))
 (segment (start 148.8 105.12) (end 148.8 79.61) (width 0.2) (layer "F.Cu") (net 23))
 (segment (start 146.19 107.73) (end 148.8 105.12) (width 0.2) (layer "F.Cu") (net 23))
 (segment (start 148.8 79.61) (end 141.73 72.54) (width 0.2) (layer "F.Cu") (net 23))
 (segment (start 150.8 99.64) (end 150.8 77.27) (width 0.2) (layer "F.Cu") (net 13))
 (segment (start 150.8 77.27) (end 155.53 72.54) (width 0.2) (layer "F.Cu") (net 13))
 (segment (start 158.89 107.73) (end 150.8 99.64) (width 0.2) (layer "F.Cu") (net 13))
 (segment (start 146.8 94.42) (end 146.8 91.41) (width 0.2) (layer "F.Cu") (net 33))
 (segment (start 146.8 91.41) (end 127.93 72.54) (width 0.2) (layer "F.Cu") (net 33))
 (segment (start 133.49 107.73) (end 146.8 94.42) (width 0.2) (layer "F.Cu") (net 33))
 (segment (start 143.135 66.105) (end 144.49 67.46) (width 0.2) (layer "F.Cu") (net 28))
 (segment (start 124.321372 113.67) (end 137.71 113.67) (width 0.2) (layer "F.Cu") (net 28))
 (segment (start 122.32 111.668628) (end 124.321372 113.67) (width 0.2) (layer "F.Cu") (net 28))
 (segment (start 137.71 113.67) (end 141.11 110.27) (width 0.2) (layer "F.Cu") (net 28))
 (segment (start 123.17 66.26) (end 122.32 67.11) (width 0.2) (layer "F.Cu") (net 28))
 (segment (start 122.32 67.11) (end 122.32 111.668628) (width 0.2) (layer "F.Cu") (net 28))
 (via (at 123.17 66.26) (size 0.6) (drill 0.3) (layers "F.Cu" "B.Cu") (free yes) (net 28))
 (via (at 143.135 66.105) (size 0.6) (drill 0.3) (layers "F.Cu" "B.Cu") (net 28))
 (segment (start 123.17 66.26) (end 142.99 66.26) (width 0.2) (layer "B.Cu") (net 28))
 (segment (start 142.99 66.26) (end 143.14 66.11) (width 0.2) (layer "B.Cu") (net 28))
 (segment (start 177.15 68.157058) (end 174.135442 65.1425) (width 0.2) (layer "F.Cu") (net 16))
 (segment (start 163.3675 65.1425) (end 161.05 67.46) (width 0.2) (layer "F.Cu") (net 16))
 (segment (start 159.33 113.25) (end 175.752942 113.25) (width 0.2) (layer "F.Cu") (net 16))
 (segment (start 156.35 110.27) (end 159.33 113.25) (width 0.2) (layer "F.Cu") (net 16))
 (segment (start 175.752942 113.25) (end 177.15 111.852942) (width 0.2) (layer "F.Cu") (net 16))
 (segment (start 177.15 111.852942) (end 177.15 68.157058) (width 0.2) (layer "F.Cu") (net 16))
 (segment (start 174.135442 65.1425) (end 163.3675 65.1425) (width 0.2) (layer "F.Cu") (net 16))
 (segment (start 163.97 107.73) (end 151.6 95.36) (width 0.2) (layer "F.Cu") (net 9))
 (segment (start 151.6 95.36) (end 151.6 81.99) (width 0.2) (layer "F.Cu") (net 9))
 (segment (start 151.6 81.99) (end 161.05 72.54) (width 0.2) (layer "F.Cu") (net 9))
 (segment (start 122.831471 65.45) (end 123.02 65.45) (width 0.2) (layer "F.Cu") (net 26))
 (segment (start 121.92 111.834314) (end 121.92 66.361471) (width 0.2) (layer "F.Cu") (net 26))
 (segment (start 143.65 110.27) (end 139.85 114.07) (width 0.2) (layer "F.Cu") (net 26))
 (segment (start 139.85 114.07) (end 124.155686 114.07) (width 0.2) (layer "F.Cu") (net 26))
 (segment (start 145.235 65.445) (end 147.25 67.46) (width 0.2) (layer "F.Cu") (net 26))
 (segment (start 121.92 66.361471) (end 122.831471 65.45) (width 0.2) (layer "F.Cu") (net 26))
 (segment (start 124.155686 114.07) (end 121.92 111.834314) (width 0.2) (layer "F.Cu") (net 26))
 (via (at 145.235 65.445) (size 0.6) (drill 0.3) (layers "F.Cu" "B.Cu") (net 26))
 (via (at 123.02 65.45) (size 0.6) (drill 0.3) (layers "F.Cu" "B.Cu") (free yes) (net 26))
 (segment (start 123.02 65.45) (end 145.24 65.45) (width 0.2) (layer "B.Cu") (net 26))
 (segment (start 175.587256 112.85) (end 176.75 111.687256) (width 0.2) (layer "F.Cu") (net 14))
 (segment (start 176.75 68.322744) (end 173.969756 65.5425) (width 0.2) (layer "F.Cu") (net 14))
 (segment (start 176.75 111.687256) (end 176.75 68.322744) (width 0.2) (layer "F.Cu") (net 14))
 (segment (start 161.47 112.85) (end 175.587256 112.85) (width 0.2) (layer "F.Cu") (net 14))
 (segment (start 173.969756 65.5425) (end 165.7275 65.5425) (width 0.2) (layer "F.Cu") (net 14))
 (segment (start 158.89 110.27) (end 161.47 112.85) (width 0.2) (layer "F.Cu") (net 14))
 (segment (start 165.7275 65.5425) (end 163.81 67.46) (width 0.2) (layer "F.Cu") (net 14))
 (segment (start 166.51 107.73) (end 152 93.22) (width 0.2) (layer "F.Cu") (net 7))
 (segment (start 152 93.22) (end 152 84.35) (width 0.2) (layer "F.Cu") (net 7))
 (segment (start 152 84.35) (end 163.81 72.54) (width 0.2) (layer "F.Cu") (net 7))
 (segment (start 153.81 107.73) (end 150 103.92) (width 0.2) (layer "F.Cu") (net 17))
 (segment (start 150 72.55) (end 150.01 72.54) (width 0.2) (layer "F.Cu") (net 17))
 (segment (start 150 103.92) (end 150 72.55) (width 0.2) (layer "F.Cu") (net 17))
 (segment (start 122.99 64.63) (end 121.15 64.63) (width 0.2) (layer "F.Cu") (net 24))
 (segment (start 147.33 64.78) (end 150.01 67.46) (width 0.2) (layer "F.Cu") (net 24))
 (segment (start 123.99 114.47) (end 141.99 114.47) (width 0.2) (layer "F.Cu") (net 24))
 (segment (start 121.15 64.63) (end 116.81 68.97) (width 0.2) (layer "F.Cu") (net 24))
 (segment (start 147.32 64.77) (end 147.33 64.78) (width 0.2) (layer "F.Cu") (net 24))
 (segment (start 116.81 107.29) (end 123.99 114.47) (width 0.2) (layer "F.Cu") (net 24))
 (segment (start 116.81 68.97) (end 116.81 107.29) (width 0.2) (layer "F.Cu") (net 24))
 (segment (start 141.99 114.47) (end 146.19 110.27) (width 0.2) (layer "F.Cu") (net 24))
 (via (at 122.99 64.63) (size 0.6) (drill 0.3) (layers "F.Cu" "B.Cu") (free yes) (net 24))
 (via (at 147.33 64.78) (size 0.6) (drill 0.3) (layers "F.Cu" "B.Cu") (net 24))
 (segment (start 147.18 64.63) (end 147.35 64.8) (width 0.2) (layer "B.Cu") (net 24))
 (segment (start 122.99 64.63) (end 147.18 64.63) (width 0.2) (layer "B.Cu") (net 24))
 (segment (start 177.95 112.184314) (end 177.95 66.9) (width 0.2) (layer "F.Cu") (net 20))
 (segment (start 176.084314 114.05) (end 177.95 112.184314) (width 0.2) (layer "F.Cu") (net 20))
 (segment (start 155.05 114.05) (end 176.084314 114.05) (width 0.2) (layer "F.Cu") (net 20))
 (segment (start 151.27 110.27) (end 155.05 114.05) (width 0.2) (layer "F.Cu") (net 20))
 (segment (start 157.19 65.8) (end 155.53 67.46) (width 0.2) (layer "F.Cu") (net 20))
 (segment (start 177.95 66.9) (end 176.85 65.8) (width 0.2) (layer "F.Cu") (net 20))
 (via (at 176.85 65.8) (size 0.6) (drill 0.3) (layers "F.Cu" "B.Cu") (free yes) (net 20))
 (via (at 157.19 65.8) (size 0.6) (drill 0.3) (layers "F.Cu" "B.Cu") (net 20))
 (segment (start 157.19 65.8) (end 176.85 65.8) (width 0.2) (layer "B.Cu") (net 20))
 (segment (start 149.2 77.25) (end 144.49 72.54) (width 0.2) (layer "F.Cu") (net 21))
 (segment (start 149.19 107.27) (end 149.19 105.295686) (width 0.2) (layer "F.Cu") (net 21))
 (segment (start 149.2 105.285686) (end 149.2 77.25) (width 0.2) (layer "F.Cu") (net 21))
 (segment (start 148.73 107.73) (end 149.19 107.27) (width 0.2) (layer "F.Cu") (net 21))
 (segment (start 149.19 105.295686) (end 149.2 105.285686) (width 0.2) (layer "F.Cu") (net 21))
 (segment (start 173.638384 66.3425) (end 175.95 68.654116) (width 0.2) (layer "F.Cu") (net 10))
 (segment (start 170.4475 66.3425) (end 173.638384 66.3425) (width 0.2) (layer "F.Cu") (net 10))
 (segment (start 175.255884 112.05) (end 165.75 112.05) (width 0.2) (layer "F.Cu") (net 10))
 (segment (start 165.75 112.05) (end 163.97 110.27) (width 0.2) (layer "F.Cu") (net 10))
 (segment (start 169.33 67.46) (end 170.4475 66.3425) (width 0.2) (layer "F.Cu") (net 10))
 (segment (start 175.95 68.654116) (end 175.95 111.355884) (width 0.2) (layer "F.Cu") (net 10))
 (segment (start 175.95 111.355884) (end 175.255884 112.05) (width 0.2) (layer "F.Cu") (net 10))
 (segment (start 175.55 111.190198) (end 175.55 70.92) (width 0.2) (layer "F.Cu") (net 8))
 (segment (start 167.89 111.65) (end 175.090198 111.65) (width 0.2) (layer "F.Cu") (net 8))
 (segment (start 175.090198 111.65) (end 175.55 111.190198) (width 0.2) (layer "F.Cu") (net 8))
 (segment (start 166.51 110.27) (end 167.89 111.65) (width 0.2) (layer "F.Cu") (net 8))
 (segment (start 175.55 70.92) (end 172.09 67.46) (width 0.2) (layer "F.Cu") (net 8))
 (segment (start 149.6 106.03) (end 149.6 74.89) (width 0.2) (layer "F.Cu") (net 19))
 (segment (start 149.6 74.89) (end 147.25 72.54) (width 0.2) (layer "F.Cu") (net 19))
 (segment (start 151.27 107.73) (end 151.27 107.7) (width 0.2) (layer "F.Cu") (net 19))
 (segment (start 151.27 107.7) (end 149.6 106.03) (width 0.2) (layer "F.Cu") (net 19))
 (segment (start 136.03 107.73) (end 147.2 96.56) (width 0.2) (layer "F.Cu") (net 31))
 (segment (start 147.2 96.56) (end 147.2 89.05) (width 0.2) (layer "F.Cu") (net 31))
 (segment (start 147.2 89.05) (end 130.69 72.54) (width 0.2) (layer "F.Cu") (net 31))
 (segment (start 136.21 67.46) (end 134.2925 65.5425) (width 0.2) (layer "F.Cu") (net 34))
 (segment (start 126.730244 65.5425) (end 123.52 68.752744) (width 0.2) (layer "F.Cu") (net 34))
 (segment (start 123.52 68.752744) (end 123.52 111.17157) (width 0.2) (layer "F.Cu") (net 34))
 (segment (start 134.2925 65.5425) (end 126.730244 65.5425) (width 0.2) (layer "F.Cu") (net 34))
 (segment (start 131.29 112.47) (end 133.49 110.27) (width 0.2) (layer "F.Cu") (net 34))
 (segment (start 123.52 111.17157) (end 124.81843 112.47) (width 0.2) (layer "F.Cu") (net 34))
 (segment (start 124.81843 112.47) (end 131.29 112.47) (width 0.2) (layer "F.Cu") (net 34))
 (segment (start 174.301128 64.7425) (end 161.0075 64.7425) (width 0.2) (layer "F.Cu") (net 18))
 (segment (start 177.55 112.018628) (end 177.55 67.991372) (width 0.2) (layer "F.Cu") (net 18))
 (segment (start 157.19 113.65) (end 175.918628 113.65) (width 0.2) (layer "F.Cu") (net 18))
 (segment (start 161.0075 64.7425) (end 158.29 67.46) (width 0.2) (layer "F.Cu") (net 18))
 (segment (start 153.81 110.27) (end 157.19 113.65) (width 0.2) (layer "F.Cu") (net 18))
 (segment (start 175.918628 113.65) (end 177.55 112.018628) (width 0.2) (layer "F.Cu") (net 18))
 (segment (start 177.55 67.991372) (end 174.301128 64.7425) (width 0.2) (layer "F.Cu") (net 18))
 (segment (start 130.95 107.73) (end 130.95 101.23) (width 0.2) (layer "F.Cu") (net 35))
 (segment (start 130.95 101.23) (end 140.13 92.05) (width 0.2) (layer "F.Cu") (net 35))
 (via (at 140.13 92.05) (size 0.6) (drill 0.3) (layers "F.Cu" "B.Cu") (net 35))
 (segment (start 158.461372 92.05) (end 170.71 79.801372) (width 0.2) (layer "B.Cu") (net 35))
 (segment (start 170.71 79.801372) (end 170.71 70) (width 0.2) (layer "B.Cu") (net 35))
 (segment (start 140.13 92.05) (end 158.461372 92.05) (width 0.2) (layer "B.Cu") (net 35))
 (segment (start 128.41 107.73) (end 128.41 101.6) (width 0.2) (layer "F.Cu") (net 37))
 (segment (start 128.41 101.6) (end 140.08 89.93) (width 0.2) (layer "F.Cu") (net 37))
 (via (at 140.08 89.93) (size 0.6) (drill 0.3) (layers "F.Cu" "B.Cu") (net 37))
 (segment (start 140.08 89.93) (end 160.015686 89.93) (width 0.2) (layer "B.Cu") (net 37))
 (segment (start 167.95 81.995686) (end 167.95 70) (width 0.2) (layer "B.Cu") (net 37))
 (segment (start 160.015686 89.93) (end 167.95 81.995686) (width 0.2) (layer "B.Cu") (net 37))
 (segment (start 156.35 107.73) (end 150.4 101.78) (width 0.2) (layer "F.Cu") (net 15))
 (segment (start 150.4 101.78) (end 150.4 74.91) (width 0.2) (layer "F.Cu") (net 15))
 (segment (start 150.4 74.91) (end 152.77 72.54) (width 0.2) (layer "F.Cu") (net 15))
 (segment (start 125.87 102.24) (end 140.08 88.03) (width 0.2) (layer "F.Cu") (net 39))
 (segment (start 125.87 107.73) (end 125.87 102.24) (width 0.2) (layer "F.Cu") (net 39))
 (via (at 140.08 88.03) (size 0.6) (drill 0.3) (layers "F.Cu" "B.Cu") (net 39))
 (segment (start 140.08 88.03) (end 161.35 88.03) (width 0.2) (layer "B.Cu") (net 39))
 (segment (start 161.35 88.03) (end 165.19 84.19) (width 0.2) (layer "B.Cu") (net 39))
 (segment (start 165.19 84.19) (end 165.19 70) (width 0.2) (layer "B.Cu") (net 39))
 (segment (start 158.39 94.5) (end 139.97 94.5) (width 0.2) (layer "B.Cu") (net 4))
 (segment (start 132.07 86.6) (end 132.07 70) (width 0.2) (layer "B.Cu") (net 4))
 (segment (start 139.97 94.5) (end 132.07 86.6) (width 0.2) (layer "B.Cu") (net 4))
 (segment (start 170.33 109.01) (end 170.33 106.44) (width 0.2) (layer "B.Cu") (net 4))
 (segment (start 171.59 110.27) (end 170.33 109.01) (width 0.2) (layer "B.Cu") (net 4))
 (segment (start 170.33 106.44) (end 158.39 94.5) (width 0.2) (layer "B.Cu") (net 4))
 (segment (start 148 100.84) (end 148 84.33) (width 0.2) (layer "F.Cu") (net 27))
 (segment (start 141.11 107.73) (end 148 100.84) (width 0.2) (layer "F.Cu") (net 27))
 (segment (start 148 84.33) (end 136.21 72.54) (width 0.2) (layer "F.Cu") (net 27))
 (segment (start 176.97 64.92) (end 179.19 64.92) (width 0.2) (layer "F.Cu") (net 22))
 (segment (start 183.19 68.92) (end 183.19 107.51) (width 0.2) (layer "F.Cu") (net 22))
 (segment (start 155.19 65.04) (end 155.2 65.04) (width 0.2) (layer "F.Cu") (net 22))
 (segment (start 155.2 65.04) (end 155.32 64.92) (width 0.2) (layer "F.Cu") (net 22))
 (segment (start 183.19 107.51) (end 176.25 114.45) (width 0.2) (layer "F.Cu") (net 22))
 (segment (start 179.19 64.92) (end 183.19 68.92) (width 0.2) (layer "F.Cu") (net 22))
 (segment (start 155.32 64.92) (end 155.31 64.92) (width 0.2) (layer "F.Cu") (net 22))
 (segment (start 176.25 114.45) (end 152.91 114.45) (width 0.2) (layer "F.Cu") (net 22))
 (segment (start 152.91 114.45) (end 148.73 110.27) (width 0.2) (layer "F.Cu") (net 22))
 (segment (start 155.31 64.92) (end 152.77 67.46) (width 0.2) (layer "F.Cu") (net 22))
 (via (at 176.97 64.92) (size 0.6) (drill 0.3) (layers "F.Cu" "B.Cu") (free yes) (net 22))
 (via (at 155.32 64.92) (size 0.6) (drill 0.3) (layers "F.Cu" "B.Cu") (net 22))
 (segment (start 155.32 64.92) (end 176.97 64.92) (width 0.2) (layer "B.Cu") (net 22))
 (segment (start 163.61 112.45) (end 175.42157 112.45) (width 0.2) (layer "F.Cu") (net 12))
 (segment (start 161.43 110.27) (end 163.61 112.45) (width 0.2) (layer "F.Cu") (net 12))
 (segment (start 173.80407 65.9425) (end 168.0875 65.9425) (width 0.2) (layer "F.Cu") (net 12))
 (segment (start 175.42157 112.45) (end 176.35 111.52157) (width 0.2) (layer "F.Cu") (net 12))
 (segment (start 176.35 68.48843) (end 173.80407 65.9425) (width 0.2) (layer "F.Cu") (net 12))
 (segment (start 176.35 111.52157) (end 176.35 68.48843) (width 0.2) (layer "F.Cu") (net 12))
 (segment (start 168.0875 65.9425) (end 166.57 67.46) (width 0.2) (layer "F.Cu") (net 12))
 (segment (start 127.01 111.67) (end 125.149802 111.67) (width 0.2) (layer "F.Cu") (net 38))
 (segment (start 125.149802 111.67) (end 124.32 110.840198) (width 0.2) (layer "F.Cu") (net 38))
 (segment (start 124.32 69.084116) (end 127.061616 66.3425) (width 0.2) (layer "F.Cu") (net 38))
 (segment (start 127.061616 66.3425) (end 129.5725 66.3425) (width 0.2) (layer "F.Cu") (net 38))
 (segment (start 129.5725 66.3425) (end 130.69 67.46) (width 0.2) (layer "F.Cu") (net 38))
 (segment (start 128.41 110.27) (end 127.01 111.67) (width 0.2) (layer "F.Cu") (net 38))
 (segment (start 124.32 110.840198) (end 124.32 69.084116) (width 0.2) (layer "F.Cu") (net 38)))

